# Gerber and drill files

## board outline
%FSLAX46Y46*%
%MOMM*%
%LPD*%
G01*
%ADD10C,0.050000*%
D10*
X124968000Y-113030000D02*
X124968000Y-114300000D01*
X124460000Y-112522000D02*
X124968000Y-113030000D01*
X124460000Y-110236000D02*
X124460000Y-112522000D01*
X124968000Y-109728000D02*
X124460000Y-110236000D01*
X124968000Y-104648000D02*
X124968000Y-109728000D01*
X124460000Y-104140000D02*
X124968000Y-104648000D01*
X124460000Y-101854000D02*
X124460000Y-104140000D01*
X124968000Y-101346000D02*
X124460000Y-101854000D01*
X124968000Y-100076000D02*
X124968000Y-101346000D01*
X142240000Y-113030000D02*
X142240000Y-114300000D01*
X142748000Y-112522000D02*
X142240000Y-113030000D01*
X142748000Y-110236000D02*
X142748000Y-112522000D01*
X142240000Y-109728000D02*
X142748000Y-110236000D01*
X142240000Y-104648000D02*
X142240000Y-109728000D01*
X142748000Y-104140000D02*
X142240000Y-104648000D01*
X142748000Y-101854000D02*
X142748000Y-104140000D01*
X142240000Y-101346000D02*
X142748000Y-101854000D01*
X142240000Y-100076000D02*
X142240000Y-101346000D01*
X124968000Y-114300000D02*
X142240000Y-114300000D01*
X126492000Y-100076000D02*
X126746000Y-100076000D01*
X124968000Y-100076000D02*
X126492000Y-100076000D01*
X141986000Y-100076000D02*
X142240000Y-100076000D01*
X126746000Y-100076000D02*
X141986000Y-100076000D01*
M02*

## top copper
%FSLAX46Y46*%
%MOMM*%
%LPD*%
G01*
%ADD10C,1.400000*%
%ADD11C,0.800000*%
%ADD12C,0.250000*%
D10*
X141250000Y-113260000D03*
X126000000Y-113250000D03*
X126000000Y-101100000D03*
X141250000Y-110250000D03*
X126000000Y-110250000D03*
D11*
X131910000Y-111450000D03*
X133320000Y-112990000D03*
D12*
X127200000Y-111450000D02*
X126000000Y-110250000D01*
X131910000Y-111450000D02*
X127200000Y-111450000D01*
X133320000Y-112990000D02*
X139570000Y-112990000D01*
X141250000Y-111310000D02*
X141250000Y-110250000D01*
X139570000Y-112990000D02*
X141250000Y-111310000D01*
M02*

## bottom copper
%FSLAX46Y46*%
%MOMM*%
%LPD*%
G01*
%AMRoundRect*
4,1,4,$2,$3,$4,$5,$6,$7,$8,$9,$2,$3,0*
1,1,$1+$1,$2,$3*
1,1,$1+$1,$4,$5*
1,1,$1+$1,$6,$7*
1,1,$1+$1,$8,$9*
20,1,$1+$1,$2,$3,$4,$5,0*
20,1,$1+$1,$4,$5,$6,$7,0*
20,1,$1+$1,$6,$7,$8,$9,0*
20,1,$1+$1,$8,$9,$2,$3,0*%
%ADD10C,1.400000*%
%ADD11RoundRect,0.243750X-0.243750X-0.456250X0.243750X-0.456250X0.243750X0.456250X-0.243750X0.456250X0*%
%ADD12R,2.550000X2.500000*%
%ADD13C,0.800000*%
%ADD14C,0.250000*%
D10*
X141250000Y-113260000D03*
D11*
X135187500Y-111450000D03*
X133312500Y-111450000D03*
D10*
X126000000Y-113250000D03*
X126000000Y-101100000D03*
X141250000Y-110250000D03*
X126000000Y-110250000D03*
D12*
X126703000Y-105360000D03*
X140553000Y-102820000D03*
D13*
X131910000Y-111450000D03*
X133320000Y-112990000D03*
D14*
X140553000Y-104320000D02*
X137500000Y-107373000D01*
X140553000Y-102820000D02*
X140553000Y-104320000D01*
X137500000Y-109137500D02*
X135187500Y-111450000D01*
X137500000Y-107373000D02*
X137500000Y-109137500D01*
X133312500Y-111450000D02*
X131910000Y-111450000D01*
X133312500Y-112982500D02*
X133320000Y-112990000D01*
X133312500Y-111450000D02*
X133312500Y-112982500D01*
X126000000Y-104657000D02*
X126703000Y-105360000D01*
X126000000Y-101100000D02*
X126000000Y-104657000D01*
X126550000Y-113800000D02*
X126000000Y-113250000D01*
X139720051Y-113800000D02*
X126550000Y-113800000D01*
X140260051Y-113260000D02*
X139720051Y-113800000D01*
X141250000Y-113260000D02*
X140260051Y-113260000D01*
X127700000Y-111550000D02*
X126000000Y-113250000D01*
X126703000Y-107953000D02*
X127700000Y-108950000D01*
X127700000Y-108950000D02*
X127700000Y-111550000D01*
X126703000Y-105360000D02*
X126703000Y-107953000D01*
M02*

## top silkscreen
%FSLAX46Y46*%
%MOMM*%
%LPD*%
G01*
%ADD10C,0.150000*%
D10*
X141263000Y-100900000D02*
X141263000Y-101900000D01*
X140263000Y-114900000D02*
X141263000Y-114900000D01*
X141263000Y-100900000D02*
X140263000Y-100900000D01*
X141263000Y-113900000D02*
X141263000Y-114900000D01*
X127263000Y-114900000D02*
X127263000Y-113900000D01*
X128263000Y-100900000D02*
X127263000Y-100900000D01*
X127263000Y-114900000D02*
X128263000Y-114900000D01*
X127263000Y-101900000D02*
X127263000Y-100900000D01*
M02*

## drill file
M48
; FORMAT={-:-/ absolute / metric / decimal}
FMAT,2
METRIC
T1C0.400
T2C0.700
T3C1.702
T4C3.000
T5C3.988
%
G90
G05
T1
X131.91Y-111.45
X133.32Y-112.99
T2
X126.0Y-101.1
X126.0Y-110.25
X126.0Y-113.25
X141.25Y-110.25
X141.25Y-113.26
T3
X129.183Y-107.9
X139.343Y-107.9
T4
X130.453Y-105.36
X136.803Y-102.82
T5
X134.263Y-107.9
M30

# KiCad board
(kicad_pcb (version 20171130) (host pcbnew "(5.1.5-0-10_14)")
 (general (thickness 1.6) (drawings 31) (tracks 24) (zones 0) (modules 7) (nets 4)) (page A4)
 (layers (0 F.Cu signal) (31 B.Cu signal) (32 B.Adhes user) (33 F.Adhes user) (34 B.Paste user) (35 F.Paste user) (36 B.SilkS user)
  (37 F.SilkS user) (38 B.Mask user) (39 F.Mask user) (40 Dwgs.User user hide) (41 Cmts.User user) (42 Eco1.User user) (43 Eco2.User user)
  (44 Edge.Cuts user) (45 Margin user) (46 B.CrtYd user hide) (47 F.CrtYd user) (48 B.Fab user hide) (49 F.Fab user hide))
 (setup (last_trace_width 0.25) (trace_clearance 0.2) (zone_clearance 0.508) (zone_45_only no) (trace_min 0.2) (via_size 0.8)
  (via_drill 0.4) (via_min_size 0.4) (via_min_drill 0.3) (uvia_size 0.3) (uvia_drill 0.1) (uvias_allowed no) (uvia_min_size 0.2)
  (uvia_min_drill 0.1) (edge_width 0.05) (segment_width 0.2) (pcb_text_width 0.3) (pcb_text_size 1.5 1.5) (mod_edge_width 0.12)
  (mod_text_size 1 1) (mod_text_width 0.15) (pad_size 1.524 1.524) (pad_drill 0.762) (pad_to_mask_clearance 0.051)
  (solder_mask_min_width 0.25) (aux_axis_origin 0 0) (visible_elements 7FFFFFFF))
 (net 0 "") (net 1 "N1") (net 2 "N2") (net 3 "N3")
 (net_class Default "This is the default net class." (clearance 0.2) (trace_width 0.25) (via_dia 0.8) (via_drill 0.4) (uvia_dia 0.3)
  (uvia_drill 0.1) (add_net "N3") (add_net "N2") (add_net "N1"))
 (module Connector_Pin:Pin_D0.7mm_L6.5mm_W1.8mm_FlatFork (layer B.Cu) (at 141.25 113.26)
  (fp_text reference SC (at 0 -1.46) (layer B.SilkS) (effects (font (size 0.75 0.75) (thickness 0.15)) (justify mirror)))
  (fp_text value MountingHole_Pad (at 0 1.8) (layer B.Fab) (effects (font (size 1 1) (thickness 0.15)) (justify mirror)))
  (pad 1 thru_hole circle (at 0 0) (size 1.4 1.4) (drill 0.7) (layers *.Cu *.Mask) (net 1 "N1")))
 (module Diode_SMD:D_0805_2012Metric (layer B.Cu) (at 134.25 111.45)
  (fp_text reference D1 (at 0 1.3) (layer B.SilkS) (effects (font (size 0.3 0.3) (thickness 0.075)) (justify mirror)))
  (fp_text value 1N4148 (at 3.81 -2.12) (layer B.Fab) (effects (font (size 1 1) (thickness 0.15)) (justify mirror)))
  (pad 2 smd roundrect (at 0.9375 0) (size 0.975 1.4) (layers B.Cu B.Paste B.Mask) (roundrect_rratio 0.25) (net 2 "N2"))
  (pad 1 smd roundrect (at -0.9375 0) (size 0.975 1.4) (layers B.Cu B.Paste B.Mask) (roundrect_rratio 0.25) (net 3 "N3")))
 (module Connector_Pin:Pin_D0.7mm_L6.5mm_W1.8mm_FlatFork (layer B.Cu) (at 126 113.25)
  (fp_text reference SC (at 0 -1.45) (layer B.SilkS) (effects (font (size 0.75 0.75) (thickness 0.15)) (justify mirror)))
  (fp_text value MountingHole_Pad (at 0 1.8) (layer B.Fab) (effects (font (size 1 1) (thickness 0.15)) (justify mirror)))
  (pad 1 thru_hole circle (at 0 0) (size 1.4 1.4) (drill 0.7) (layers *.Cu *.Mask) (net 1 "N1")))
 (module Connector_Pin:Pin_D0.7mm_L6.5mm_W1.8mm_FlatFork (layer B.Cu) (at 126 101.1)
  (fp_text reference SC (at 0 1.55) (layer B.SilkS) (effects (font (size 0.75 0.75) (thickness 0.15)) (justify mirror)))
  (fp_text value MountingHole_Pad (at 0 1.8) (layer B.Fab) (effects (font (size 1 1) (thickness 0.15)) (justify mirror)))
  (pad 1 thru_hole circle (at 0 0) (size 1.4 1.4) (drill 0.7) (layers *.Cu *.Mask) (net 1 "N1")))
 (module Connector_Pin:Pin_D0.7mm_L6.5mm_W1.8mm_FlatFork (layer B.Cu) (at 141.25 110.25)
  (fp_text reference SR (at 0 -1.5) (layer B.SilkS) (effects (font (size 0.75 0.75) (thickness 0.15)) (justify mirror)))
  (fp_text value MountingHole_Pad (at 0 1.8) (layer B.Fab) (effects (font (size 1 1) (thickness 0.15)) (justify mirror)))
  (pad 1 thru_hole circle (at 0 0) (size 1.4 1.4) (drill 0.7) (layers *.Cu *.Mask) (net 3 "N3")))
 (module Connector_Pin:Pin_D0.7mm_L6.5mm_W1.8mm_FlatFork (layer B.Cu) (at 126 110.25)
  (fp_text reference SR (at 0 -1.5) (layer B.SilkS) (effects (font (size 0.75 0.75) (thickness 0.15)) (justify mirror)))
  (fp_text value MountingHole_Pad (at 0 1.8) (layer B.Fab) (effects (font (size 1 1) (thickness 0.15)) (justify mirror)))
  (pad 1 thru_hole circle (at 0 0) (size 1.4 1.4) (drill 0.7) (layers *.Cu *.Mask) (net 3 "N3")))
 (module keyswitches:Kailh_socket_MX (layer F.Cu) (at 134.263 107.9)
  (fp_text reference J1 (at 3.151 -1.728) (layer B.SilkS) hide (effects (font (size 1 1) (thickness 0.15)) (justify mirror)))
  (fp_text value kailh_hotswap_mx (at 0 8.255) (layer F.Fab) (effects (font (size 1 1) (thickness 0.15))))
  (fp_line (start 7 -7) (end 7 -6) (layer F.SilkS) (width 0.15)) (fp_line (start 6 7) (end 7 7) (layer F.SilkS) (width 0.15))
  (fp_line (start 7 -7) (end 6 -7) (layer F.SilkS) (width 0.15)) (fp_line (start 7 6) (end 7 7) (layer F.SilkS) (width 0.15))
  (fp_line (start -7 7) (end -7 6) (layer F.SilkS) (width 0.15))
  (fp_line (start -6 -7) (end -7 -7) (layer F.SilkS) (width 0.15))
  (fp_line (start -7 7) (end -6 7) (layer F.SilkS) (width 0.15))
  (fp_line (start -7 -6) (end -7 -7) (layer F.SilkS) (width 0.15))
  (pad 2 smd rect (at -7.56 -2.54) (size 2.55 2.5) (layers B.Cu B.Paste B.Mask) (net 1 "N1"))
  (pad "" np_thru_hole circle (at -5.08 0) (size 1.7018 1.7018) (drill 1.7018) (layers *.Cu *.Mask))
  (pad "" np_thru_hole circle (at 5.08 0) (size 1.7018 1.7018) (drill 1.7018) (layers *.Cu *.Mask))
  (pad "" np_thru_hole circle (at 0 0) (size 3.9878 3.9878) (drill 3.9878) (layers *.Cu *.Mask))
  (pad "" np_thru_hole circle (at -3.81 -2.54) (size 3 3) (drill 3) (layers *.Cu *.Mask))
  (pad "" np_thru_hole circle (at 2.54 -5.08) (size 3 3) (drill 3) (layers *.Cu *.Mask))
  (pad 1 smd rect (at 6.29 -5.08) (size 2.55 2.5) (layers B.Cu B.Paste B.Mask) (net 2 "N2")))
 (gr_line (start 124.968 113.03) (end 124.968 114.3) (layer Edge.Cuts) (width 0.05))
 (gr_line (start 124.46 112.522) (end 124.968 113.03) (layer Edge.Cuts) (width 0.05))
 (gr_line (start 124.46 110.236) (end 124.46 112.522) (layer Edge.Cuts) (width 0.05))
 (gr_line (start 124.968 109.728) (end 124.46 110.236) (layer Edge.Cuts) (width 0.05))
 (gr_line (start 124.968 104.648) (end 124.968 109.728) (layer Edge.Cuts) (width 0.05))
 (gr_line (start 124.46 104.14) (end 124.968 104.648) (layer Edge.Cuts) (width 0.05))
 (gr_line (start 124.46 101.854) (end 124.46 104.14) (layer Edge.Cuts) (width 0.05))
 (gr_line (start 124.968 101.346) (end 124.46 101.854) (layer Edge.Cuts) (width 0.05))
 (gr_line (start 124.968 100.076) (end 124.968 101.346) (layer Edge.Cuts) (width 0.05))
 (gr_line (start 142.24 113.03) (end 142.24 114.3) (layer Edge.Cuts) (width 0.05))
 (gr_line (start 142.748 112.522) (end 142.24 113.03) (layer Edge.Cuts) (width 0.05))
 (gr_line (start 142.748 110.236) (end 142.748 112.522) (layer Edge.Cuts) (width 0.05))
 (gr_line (start 142.24 109.728) (end 142.748 110.236) (layer Edge.Cuts) (width 0.05))
 (gr_line (start 142.24 104.648) (end 142.24 109.728) (layer Edge.Cuts) (width 0.05))
 (gr_line (start 142.748 104.14) (end 142.24 104.648) (layer Edge.Cuts) (width 0.05))
 (gr_line (start 142.748 101.854) (end 142.748 104.14) (layer Edge.Cuts) (width 0.05))
 (gr_line (start 142.24 101.346) (end 142.748 101.854) (layer Edge.Cuts) (width 0.05))
 (gr_line (start 142.24 100.076) (end 142.24 101.346) (layer Edge.Cuts) (width 0.05))
 (gr_line (start 124.968 114.3) (end 142.24 114.3) (layer Edge.Cuts) (width 0.05))
 (gr_line (start 126.492 100.076) (end 126.746 100.076) (layer Edge.Cuts) (width 0.05))
 (gr_line (start 124.968 100.076) (end 126.492 100.076) (layer Edge.Cuts) (width 0.05))
 (gr_line (start 141.986 100.076) (end 142.24 100.076) (layer Edge.Cuts) (width 0.05))
 (gr_line (start 126.746 100.076) (end 141.986 100.076) (layer Edge.Cuts) (width 0.05))
 (segment (start 140.553 104.32) (end 137.5 107.373) (width 0.25) (layer B.Cu) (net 2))
 (segment (start 140.553 102.82) (end 140.553 104.32) (width 0.25) (layer B.Cu) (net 2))
 (segment (start 137.5 109.1375) (end 135.1875 111.45) (width 0.25) (layer B.Cu) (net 2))
 (segment (start 137.5 107.373) (end 137.5 109.1375) (width 0.25) (layer B.Cu) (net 2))
 (via (at 131.91 111.45) (size 0.8) (drill 0.4) (layers F.Cu B.Cu) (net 3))
 (segment (start 133.3125 111.45) (end 131.91 111.45) (width 0.25) (layer B.Cu) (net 3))
 (segment (start 127.2 111.45) (end 126 110.25) (width 0.25) (layer F.Cu) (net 3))
 (segment (start 131.91 111.45) (end 127.2 111.45) (width 0.25) (layer F.Cu) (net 3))
 (via (at 133.32 112.99) (size 0.8) (drill 0.4) (layers F.Cu B.Cu) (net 3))
 (segment (start 133.3125 112.9825) (end 133.32 112.99) (width 0.25) (layer B.Cu) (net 3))
 (segment (start 133.3125 111.45) (end 133.3125 112.9825) (width 0.25) (layer B.Cu) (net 3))
 (segment (start 133.32 112.99) (end 139.57 112.99) (width 0.25) (layer F.Cu) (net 3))
 (segment (start 141.25 111.31) (end 141.25 110.25) (width 0.25) (layer F.Cu) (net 3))
 (segment (start 139.57 112.99) (end 141.25 111.31) (width 0.25) (layer F.Cu) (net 3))
 (segment (start 126 104.657) (end 126.703 105.36) (width 0.25) (layer B.Cu) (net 1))
 (segment (start 126 101.1) (end 126 104.657) (width 0.25) (layer B.Cu) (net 1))
 (segment (start 126.55 113.8) (end 126 113.25) (width 0.25) (layer B.Cu) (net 1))
 (segment (start 139.720051 113.8) (end 126.55 113.8) (width 0.25) (layer B.Cu) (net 1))
 (segment (start 140.260051 113.26) (end 139.720051 113.8) (width 0.25) (layer B.Cu) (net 1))
 (segment (start 141.25 113.26) (end 140.260051 113.26) (width 0.25) (layer B.Cu) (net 1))
 (segment (start 127.7 111.55) (end 126 113.25) (width 0.25) (layer B.Cu) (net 1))
 (segment (start 126.703 107.953) (end 127.7 108.95) (width 0.25) (layer B.Cu) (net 1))
 (segment (start 127.7 108.95) (end 127.7 111.55) (width 0.25) (layer B.Cu) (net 1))
 (segment (start 126.703 105.36) (end 126.703 107.953) (width 0.25) (layer B.Cu) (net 1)))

